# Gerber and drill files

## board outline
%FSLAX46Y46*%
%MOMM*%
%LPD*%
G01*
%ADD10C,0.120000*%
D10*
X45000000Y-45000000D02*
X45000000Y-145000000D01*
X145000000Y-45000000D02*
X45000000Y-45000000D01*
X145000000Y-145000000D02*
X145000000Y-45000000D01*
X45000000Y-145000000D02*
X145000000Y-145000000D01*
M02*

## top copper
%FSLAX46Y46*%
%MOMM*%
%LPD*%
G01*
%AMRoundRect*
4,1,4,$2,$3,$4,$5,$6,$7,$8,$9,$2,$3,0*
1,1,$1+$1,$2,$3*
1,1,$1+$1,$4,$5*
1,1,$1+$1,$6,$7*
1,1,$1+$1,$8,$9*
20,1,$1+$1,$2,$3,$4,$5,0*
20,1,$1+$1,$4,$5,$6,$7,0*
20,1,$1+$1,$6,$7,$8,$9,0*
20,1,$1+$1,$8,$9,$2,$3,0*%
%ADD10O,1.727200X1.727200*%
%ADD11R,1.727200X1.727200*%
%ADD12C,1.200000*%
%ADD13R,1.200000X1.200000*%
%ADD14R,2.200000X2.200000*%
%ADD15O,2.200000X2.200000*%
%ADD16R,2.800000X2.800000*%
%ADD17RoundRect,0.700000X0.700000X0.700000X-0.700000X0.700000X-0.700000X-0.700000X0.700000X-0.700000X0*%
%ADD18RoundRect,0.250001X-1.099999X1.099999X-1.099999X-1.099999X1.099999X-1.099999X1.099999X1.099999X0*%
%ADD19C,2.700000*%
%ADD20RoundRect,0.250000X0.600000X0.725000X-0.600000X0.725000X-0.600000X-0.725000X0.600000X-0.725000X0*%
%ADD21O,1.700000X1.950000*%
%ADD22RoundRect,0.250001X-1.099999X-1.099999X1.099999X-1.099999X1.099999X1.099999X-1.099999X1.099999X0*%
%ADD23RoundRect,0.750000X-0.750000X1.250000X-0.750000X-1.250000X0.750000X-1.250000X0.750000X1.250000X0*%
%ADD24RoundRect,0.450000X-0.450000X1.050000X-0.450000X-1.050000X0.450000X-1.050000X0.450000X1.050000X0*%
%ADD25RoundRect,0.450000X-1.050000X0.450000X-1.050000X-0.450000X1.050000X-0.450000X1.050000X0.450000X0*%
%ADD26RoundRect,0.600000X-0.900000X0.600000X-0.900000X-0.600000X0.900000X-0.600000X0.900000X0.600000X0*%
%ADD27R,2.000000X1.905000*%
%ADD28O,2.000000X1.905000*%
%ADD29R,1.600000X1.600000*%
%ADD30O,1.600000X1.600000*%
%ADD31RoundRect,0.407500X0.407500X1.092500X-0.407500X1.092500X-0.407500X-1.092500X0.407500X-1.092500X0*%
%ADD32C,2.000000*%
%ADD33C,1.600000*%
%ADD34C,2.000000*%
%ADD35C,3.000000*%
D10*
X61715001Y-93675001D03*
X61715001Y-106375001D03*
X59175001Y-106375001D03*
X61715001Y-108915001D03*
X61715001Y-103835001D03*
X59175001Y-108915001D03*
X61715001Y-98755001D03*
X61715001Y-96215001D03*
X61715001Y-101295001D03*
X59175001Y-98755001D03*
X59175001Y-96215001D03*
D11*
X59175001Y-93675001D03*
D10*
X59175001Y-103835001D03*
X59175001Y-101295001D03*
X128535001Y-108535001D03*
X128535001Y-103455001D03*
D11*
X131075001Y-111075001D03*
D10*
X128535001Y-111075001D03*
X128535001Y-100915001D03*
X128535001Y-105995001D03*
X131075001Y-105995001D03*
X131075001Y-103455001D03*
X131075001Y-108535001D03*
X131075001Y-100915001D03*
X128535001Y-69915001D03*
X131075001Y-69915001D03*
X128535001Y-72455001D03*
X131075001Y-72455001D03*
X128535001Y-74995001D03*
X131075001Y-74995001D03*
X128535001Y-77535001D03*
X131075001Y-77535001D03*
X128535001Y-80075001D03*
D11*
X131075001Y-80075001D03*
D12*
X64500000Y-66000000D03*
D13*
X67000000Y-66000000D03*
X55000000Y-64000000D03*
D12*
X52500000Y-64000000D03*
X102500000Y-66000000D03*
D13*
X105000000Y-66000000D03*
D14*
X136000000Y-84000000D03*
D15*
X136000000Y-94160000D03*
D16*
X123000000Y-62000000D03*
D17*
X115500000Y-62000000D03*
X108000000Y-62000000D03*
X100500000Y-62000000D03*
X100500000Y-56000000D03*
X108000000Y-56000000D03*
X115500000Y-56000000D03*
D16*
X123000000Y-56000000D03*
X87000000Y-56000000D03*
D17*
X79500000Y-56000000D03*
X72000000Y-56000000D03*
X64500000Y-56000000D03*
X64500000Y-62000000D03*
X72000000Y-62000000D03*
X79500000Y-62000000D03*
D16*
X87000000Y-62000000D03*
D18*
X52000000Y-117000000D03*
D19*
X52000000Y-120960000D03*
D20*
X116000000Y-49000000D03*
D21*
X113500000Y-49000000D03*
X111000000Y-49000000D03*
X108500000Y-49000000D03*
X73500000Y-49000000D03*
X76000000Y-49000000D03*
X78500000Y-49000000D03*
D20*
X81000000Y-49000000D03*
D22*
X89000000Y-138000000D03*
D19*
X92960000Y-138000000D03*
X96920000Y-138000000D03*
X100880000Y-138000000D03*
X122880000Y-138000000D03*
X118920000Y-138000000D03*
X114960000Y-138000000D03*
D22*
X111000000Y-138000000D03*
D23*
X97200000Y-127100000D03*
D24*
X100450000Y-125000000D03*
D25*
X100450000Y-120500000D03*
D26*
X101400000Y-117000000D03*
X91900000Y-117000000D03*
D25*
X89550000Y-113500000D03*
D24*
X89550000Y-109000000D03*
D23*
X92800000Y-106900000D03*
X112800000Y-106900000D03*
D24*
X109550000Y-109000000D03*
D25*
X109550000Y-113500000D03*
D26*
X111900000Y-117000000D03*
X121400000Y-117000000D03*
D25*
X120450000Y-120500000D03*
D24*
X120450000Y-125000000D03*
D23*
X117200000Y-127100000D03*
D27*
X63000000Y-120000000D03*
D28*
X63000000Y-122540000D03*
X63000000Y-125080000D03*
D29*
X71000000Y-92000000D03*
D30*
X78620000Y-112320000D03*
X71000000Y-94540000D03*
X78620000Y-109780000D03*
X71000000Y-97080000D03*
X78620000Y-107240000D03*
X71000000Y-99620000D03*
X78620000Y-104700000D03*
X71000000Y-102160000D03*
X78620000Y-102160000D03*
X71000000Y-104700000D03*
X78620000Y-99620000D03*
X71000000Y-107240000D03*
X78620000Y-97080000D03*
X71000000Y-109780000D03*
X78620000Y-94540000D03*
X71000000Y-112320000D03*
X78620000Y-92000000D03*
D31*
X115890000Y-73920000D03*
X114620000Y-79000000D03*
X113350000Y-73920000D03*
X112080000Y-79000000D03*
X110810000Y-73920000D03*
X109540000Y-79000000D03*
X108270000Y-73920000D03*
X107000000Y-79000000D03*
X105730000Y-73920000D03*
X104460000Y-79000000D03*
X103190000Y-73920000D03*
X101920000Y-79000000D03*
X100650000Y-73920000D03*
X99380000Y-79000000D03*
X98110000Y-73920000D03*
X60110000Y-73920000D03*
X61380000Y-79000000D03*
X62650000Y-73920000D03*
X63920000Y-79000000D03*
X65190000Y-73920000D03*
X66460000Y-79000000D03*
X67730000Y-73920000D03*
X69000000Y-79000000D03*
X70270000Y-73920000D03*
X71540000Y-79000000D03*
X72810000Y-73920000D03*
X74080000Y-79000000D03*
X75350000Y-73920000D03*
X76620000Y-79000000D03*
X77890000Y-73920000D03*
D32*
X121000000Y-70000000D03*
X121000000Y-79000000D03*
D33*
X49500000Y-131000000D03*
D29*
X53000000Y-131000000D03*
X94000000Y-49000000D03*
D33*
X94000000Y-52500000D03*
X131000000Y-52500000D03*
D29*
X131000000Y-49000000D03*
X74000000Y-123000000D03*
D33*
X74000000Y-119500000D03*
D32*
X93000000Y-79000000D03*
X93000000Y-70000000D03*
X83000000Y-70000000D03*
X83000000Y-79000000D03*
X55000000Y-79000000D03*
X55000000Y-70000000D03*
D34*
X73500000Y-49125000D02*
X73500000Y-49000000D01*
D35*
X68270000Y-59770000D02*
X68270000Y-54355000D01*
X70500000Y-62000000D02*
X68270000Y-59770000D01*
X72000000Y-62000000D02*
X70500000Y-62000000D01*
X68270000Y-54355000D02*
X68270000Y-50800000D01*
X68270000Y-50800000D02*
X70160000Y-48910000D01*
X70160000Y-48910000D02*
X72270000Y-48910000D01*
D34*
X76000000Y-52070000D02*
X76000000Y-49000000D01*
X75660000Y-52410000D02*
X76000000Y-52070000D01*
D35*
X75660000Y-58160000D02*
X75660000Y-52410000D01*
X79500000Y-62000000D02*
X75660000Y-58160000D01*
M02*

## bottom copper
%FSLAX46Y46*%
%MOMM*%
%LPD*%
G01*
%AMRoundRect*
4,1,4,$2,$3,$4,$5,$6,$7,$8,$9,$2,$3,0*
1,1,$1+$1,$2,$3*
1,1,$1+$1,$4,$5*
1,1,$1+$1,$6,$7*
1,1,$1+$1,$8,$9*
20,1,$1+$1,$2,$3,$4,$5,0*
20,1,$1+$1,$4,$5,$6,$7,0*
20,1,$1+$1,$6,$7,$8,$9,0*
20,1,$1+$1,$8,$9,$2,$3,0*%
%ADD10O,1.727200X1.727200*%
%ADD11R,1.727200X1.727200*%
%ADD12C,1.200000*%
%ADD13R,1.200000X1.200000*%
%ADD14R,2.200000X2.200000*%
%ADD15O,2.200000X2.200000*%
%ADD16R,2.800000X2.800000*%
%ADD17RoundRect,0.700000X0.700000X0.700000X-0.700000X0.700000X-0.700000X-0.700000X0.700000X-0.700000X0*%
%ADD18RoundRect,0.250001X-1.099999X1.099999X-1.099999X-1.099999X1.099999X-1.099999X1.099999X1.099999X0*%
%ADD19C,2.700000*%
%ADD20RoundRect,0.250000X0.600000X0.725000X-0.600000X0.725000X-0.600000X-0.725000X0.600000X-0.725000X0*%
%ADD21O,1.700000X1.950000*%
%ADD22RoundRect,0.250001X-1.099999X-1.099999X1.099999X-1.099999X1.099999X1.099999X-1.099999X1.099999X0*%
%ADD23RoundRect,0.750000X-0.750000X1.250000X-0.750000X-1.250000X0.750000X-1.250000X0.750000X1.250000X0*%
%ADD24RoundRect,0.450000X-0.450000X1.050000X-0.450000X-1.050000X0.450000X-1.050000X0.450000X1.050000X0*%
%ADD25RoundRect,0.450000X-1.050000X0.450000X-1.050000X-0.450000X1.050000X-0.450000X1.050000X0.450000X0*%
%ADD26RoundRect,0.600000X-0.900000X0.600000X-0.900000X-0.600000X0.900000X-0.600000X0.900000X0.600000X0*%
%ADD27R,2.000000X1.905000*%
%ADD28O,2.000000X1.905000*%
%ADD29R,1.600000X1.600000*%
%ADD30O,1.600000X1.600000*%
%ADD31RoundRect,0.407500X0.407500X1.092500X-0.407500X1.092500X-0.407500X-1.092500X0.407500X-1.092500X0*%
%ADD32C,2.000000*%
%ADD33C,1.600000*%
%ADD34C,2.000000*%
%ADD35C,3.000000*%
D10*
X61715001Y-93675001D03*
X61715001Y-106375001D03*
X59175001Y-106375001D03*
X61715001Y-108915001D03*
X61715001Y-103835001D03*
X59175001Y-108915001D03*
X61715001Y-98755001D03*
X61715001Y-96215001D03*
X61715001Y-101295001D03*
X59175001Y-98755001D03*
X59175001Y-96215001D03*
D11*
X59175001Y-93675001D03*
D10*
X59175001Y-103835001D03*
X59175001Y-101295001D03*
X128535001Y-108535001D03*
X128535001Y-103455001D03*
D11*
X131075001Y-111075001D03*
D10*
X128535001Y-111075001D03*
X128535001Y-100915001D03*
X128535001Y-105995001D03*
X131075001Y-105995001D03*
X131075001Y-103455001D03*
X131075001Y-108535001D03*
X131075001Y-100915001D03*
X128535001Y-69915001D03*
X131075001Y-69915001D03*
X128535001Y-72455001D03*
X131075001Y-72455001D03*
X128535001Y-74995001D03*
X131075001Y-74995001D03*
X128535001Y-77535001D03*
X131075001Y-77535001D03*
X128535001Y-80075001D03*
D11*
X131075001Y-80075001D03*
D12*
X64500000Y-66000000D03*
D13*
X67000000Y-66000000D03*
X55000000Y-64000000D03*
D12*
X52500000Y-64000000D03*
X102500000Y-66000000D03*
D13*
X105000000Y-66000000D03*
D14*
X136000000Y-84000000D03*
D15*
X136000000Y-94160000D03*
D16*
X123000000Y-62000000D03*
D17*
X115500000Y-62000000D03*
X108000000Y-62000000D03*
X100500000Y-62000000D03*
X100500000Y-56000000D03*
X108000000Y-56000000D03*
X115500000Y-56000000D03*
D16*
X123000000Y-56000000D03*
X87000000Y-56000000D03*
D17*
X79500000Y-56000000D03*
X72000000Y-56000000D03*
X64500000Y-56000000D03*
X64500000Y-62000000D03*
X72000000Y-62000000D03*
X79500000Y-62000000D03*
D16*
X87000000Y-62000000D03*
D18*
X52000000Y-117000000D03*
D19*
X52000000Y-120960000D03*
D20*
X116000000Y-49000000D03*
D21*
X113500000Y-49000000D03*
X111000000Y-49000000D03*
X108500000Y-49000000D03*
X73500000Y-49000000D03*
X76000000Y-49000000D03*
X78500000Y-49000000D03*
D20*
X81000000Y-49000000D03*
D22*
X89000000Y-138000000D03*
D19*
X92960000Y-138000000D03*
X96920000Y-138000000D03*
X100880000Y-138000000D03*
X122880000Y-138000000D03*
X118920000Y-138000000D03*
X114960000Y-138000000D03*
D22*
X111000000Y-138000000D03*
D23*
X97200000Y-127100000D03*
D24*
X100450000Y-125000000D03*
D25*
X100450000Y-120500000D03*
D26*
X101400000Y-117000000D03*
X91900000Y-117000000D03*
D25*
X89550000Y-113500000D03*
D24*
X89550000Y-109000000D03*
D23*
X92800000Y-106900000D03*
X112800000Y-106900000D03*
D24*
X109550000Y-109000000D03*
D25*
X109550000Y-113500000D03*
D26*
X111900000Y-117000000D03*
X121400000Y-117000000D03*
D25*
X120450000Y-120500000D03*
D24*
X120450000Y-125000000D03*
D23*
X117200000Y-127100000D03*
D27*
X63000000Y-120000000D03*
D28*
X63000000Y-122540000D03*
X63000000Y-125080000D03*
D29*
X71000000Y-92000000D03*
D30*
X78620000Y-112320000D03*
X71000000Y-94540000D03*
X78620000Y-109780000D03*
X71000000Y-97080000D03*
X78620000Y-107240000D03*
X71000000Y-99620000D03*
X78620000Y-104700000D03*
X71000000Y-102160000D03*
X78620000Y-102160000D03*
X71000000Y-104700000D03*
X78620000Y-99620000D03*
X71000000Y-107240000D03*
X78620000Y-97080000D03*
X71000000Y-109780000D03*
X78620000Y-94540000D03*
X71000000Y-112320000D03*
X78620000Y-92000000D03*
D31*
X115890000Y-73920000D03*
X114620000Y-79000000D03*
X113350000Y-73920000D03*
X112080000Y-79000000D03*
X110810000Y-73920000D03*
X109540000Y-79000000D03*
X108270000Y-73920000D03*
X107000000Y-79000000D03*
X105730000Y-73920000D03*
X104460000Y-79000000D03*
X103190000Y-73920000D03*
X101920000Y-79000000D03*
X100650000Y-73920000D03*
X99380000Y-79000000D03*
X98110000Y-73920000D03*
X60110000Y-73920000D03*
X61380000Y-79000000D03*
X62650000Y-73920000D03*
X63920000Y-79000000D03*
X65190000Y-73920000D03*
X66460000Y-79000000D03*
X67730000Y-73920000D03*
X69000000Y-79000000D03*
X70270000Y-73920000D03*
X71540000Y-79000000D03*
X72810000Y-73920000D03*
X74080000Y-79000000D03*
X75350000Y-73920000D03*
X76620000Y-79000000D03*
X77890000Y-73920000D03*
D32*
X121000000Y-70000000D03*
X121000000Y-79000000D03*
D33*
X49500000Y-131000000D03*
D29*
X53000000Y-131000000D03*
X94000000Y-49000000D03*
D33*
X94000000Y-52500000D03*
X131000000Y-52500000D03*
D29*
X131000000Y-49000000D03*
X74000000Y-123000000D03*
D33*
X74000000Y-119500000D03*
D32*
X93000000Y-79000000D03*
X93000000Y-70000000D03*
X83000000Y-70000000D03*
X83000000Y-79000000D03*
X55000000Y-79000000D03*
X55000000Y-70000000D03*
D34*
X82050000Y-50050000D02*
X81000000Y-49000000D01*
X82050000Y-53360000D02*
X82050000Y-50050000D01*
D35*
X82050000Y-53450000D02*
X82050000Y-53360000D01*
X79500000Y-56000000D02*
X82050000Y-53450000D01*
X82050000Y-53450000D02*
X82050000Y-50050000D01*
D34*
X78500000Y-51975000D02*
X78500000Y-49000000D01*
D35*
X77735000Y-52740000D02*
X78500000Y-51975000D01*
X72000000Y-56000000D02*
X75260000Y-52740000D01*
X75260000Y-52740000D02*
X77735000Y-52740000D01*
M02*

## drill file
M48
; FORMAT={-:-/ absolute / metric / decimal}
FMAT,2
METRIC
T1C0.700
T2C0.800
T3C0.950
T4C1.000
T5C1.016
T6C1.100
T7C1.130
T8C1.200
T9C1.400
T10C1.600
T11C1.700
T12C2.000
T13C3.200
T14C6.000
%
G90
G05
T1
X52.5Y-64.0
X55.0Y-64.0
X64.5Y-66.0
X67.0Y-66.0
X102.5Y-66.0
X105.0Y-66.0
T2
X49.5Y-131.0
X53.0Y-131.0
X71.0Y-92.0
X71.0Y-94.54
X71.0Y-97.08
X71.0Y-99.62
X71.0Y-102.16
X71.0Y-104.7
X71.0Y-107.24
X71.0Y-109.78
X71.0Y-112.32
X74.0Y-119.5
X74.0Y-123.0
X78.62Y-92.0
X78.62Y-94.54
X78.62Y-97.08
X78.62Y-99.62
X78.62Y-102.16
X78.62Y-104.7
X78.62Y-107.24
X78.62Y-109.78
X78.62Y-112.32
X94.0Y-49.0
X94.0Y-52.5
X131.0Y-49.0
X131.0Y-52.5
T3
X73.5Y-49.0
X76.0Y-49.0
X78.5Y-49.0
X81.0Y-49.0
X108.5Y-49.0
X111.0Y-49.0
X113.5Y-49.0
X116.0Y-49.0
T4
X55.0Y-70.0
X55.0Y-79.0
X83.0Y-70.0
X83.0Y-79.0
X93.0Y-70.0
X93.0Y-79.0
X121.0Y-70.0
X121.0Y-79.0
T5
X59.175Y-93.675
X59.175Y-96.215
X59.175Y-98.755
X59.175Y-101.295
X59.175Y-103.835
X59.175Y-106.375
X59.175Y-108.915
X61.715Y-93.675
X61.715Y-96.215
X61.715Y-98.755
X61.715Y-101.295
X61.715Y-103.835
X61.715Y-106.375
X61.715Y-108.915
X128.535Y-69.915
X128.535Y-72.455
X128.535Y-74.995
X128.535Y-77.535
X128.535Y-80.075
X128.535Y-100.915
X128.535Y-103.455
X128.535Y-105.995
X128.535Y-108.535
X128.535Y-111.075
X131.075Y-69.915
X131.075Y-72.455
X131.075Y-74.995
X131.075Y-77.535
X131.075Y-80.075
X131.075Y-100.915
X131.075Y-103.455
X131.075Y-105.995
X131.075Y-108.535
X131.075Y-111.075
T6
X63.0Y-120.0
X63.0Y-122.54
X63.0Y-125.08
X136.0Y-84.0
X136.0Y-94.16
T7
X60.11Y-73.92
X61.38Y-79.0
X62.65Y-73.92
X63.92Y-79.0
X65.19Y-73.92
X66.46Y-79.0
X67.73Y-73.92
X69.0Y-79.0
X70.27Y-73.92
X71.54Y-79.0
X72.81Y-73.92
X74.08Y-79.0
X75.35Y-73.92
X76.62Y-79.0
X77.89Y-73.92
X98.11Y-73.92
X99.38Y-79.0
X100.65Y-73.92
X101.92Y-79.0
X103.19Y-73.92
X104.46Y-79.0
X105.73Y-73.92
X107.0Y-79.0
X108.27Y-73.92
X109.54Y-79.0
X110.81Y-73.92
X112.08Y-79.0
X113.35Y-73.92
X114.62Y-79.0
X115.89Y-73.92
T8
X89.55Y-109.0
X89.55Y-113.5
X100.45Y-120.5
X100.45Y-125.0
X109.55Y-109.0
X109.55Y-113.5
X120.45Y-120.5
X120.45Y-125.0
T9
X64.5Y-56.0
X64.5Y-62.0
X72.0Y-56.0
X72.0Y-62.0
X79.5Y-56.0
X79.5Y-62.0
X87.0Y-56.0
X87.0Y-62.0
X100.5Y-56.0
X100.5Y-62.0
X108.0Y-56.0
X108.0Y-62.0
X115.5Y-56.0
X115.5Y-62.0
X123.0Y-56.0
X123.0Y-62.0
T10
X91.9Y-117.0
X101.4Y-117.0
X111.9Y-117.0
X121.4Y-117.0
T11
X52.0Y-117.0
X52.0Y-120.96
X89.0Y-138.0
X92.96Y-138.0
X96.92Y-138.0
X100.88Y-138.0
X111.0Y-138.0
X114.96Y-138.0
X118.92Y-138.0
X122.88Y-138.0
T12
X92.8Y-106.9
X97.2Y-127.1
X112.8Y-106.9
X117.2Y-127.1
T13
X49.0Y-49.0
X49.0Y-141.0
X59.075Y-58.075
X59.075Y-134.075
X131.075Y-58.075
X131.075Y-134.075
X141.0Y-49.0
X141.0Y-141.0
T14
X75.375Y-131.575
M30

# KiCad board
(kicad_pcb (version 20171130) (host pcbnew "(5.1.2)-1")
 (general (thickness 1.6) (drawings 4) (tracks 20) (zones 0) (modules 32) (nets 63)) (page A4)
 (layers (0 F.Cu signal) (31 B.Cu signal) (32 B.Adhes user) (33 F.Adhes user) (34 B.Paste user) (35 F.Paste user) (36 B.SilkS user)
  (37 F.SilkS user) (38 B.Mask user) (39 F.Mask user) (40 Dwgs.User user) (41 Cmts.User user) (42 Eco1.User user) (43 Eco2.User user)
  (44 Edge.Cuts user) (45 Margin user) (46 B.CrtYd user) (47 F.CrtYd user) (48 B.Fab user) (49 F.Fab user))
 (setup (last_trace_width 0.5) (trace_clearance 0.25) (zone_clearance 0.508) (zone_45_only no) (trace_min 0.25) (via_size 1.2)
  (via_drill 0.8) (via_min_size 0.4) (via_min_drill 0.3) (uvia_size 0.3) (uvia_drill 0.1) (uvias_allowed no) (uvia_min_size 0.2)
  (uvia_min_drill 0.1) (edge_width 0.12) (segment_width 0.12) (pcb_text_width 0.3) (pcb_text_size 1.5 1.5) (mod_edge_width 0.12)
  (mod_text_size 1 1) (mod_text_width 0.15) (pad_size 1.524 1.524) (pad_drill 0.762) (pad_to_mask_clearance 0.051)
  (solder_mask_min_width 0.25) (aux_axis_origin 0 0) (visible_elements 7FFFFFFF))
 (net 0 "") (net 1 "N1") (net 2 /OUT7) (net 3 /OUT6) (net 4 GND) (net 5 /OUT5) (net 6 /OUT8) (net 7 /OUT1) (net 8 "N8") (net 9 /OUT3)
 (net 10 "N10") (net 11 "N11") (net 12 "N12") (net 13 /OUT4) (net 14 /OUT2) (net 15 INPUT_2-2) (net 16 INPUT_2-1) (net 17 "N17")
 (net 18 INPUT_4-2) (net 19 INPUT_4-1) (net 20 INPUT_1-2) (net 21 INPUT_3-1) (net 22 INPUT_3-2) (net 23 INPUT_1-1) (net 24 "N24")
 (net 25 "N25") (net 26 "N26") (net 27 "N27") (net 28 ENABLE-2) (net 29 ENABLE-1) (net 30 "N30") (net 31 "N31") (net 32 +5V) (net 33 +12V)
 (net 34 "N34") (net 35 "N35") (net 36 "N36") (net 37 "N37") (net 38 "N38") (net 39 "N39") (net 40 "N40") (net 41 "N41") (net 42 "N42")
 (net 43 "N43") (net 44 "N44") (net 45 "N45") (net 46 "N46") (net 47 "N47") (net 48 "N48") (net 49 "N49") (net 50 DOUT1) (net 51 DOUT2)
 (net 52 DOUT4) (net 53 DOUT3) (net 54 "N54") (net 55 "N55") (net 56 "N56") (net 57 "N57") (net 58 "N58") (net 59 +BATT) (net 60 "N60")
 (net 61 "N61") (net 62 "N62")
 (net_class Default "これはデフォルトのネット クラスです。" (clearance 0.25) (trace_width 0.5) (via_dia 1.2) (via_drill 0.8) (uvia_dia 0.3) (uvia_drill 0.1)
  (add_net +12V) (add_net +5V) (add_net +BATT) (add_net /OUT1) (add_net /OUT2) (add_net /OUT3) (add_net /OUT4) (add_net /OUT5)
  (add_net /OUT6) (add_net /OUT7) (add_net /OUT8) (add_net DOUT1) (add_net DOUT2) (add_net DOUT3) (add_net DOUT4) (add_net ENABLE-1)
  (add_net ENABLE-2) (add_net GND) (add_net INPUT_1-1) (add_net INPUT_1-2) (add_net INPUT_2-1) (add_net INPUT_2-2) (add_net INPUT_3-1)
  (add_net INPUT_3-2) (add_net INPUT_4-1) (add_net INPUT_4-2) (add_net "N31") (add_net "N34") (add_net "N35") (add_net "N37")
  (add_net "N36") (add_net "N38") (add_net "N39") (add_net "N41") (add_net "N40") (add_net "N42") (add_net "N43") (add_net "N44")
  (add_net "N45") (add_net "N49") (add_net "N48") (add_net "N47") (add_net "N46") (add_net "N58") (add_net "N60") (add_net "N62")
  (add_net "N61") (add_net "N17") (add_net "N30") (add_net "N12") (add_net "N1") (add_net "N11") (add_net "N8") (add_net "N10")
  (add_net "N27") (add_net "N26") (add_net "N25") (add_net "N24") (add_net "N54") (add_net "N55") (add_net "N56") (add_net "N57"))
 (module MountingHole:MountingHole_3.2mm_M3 (layer F.Cu) (at 141 49)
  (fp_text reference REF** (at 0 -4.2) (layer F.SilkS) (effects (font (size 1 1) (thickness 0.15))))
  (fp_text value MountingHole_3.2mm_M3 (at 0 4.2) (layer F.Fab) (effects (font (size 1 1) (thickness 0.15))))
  (pad 1 np_thru_hole circle (at 0 0) (size 3.2 3.2) (drill 3.2) (layers *.Cu *.Mask)))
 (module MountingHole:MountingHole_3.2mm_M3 (layer F.Cu) (at 141 141)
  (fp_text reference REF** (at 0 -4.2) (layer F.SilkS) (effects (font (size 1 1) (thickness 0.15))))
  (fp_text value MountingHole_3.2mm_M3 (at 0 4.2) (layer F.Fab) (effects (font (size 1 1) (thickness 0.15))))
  (pad 1 np_thru_hole circle (at 0 0) (size 3.2 3.2) (drill 3.2) (layers *.Cu *.Mask)))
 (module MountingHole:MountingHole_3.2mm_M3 (layer F.Cu) (at 49 141)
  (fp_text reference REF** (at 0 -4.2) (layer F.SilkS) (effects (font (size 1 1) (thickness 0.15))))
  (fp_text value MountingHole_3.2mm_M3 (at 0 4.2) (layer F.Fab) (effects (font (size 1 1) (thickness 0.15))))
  (pad 1 np_thru_hole circle (at 0 0) (size 3.2 3.2) (drill 3.2) (layers *.Cu *.Mask)))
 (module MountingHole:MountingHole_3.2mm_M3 (layer F.Cu) (at 49 49)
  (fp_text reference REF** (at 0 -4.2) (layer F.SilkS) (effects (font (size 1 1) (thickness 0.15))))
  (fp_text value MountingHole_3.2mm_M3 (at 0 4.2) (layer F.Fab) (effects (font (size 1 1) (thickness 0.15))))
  (pad 1 np_thru_hole circle (at 0 0) (size 3.2 3.2) (drill 3.2) (layers *.Cu *.Mask)))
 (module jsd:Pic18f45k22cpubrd (layer F.Cu) (at 59.075001 58.075001)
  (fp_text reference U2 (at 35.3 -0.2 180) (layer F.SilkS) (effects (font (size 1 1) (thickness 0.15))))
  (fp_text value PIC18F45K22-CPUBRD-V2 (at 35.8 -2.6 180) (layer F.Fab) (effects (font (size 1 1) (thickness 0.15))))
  (pad "" np_thru_hole circle (at 16.3 73.5) (size 6 6) (drill 6) (layers *.Cu *.Mask))
  (pad "" np_thru_hole circle (at 72 76) (size 3.2 3.2) (drill 3.2) (layers *.Cu *.Mask))
  (pad "" np_thru_hole circle (at 72 0) (size 3.2 3.2) (drill 3.2) (layers *.Cu *.Mask))
  (pad "" np_thru_hole circle (at 0 0) (size 3.2 3.2) (drill 3.2) (layers *.Cu *.Mask))
  (pad "" np_thru_hole circle (at 0 76) (size 3.2 3.2) (drill 3.2) (layers *.Cu *.Mask))
  (pad 22 thru_hole oval (at 2.64 35.6) (size 1.7272 1.7272) (drill 1.016) (layers *.Cu *.Mask) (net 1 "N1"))
  (pad 32 thru_hole oval (at 2.64 48.3) (size 1.7272 1.7272) (drill 1.016) (layers *.Cu *.Mask) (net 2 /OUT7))
  (pad 31 thru_hole oval (at 0.1 48.3) (size 1.7272 1.7272) (drill 1.016) (layers *.Cu *.Mask) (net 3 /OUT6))
  (pad 34 thru_hole oval (at 2.64 50.84) (size 1.7272 1.7272) (drill 1.016) (layers *.Cu *.Mask) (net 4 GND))
  (pad 30 thru_hole oval (at 2.64 45.76) (size 1.7272 1.7272) (drill 1.016) (layers *.Cu *.Mask) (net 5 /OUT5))
  (pad 33 thru_hole oval (at 0.1 50.84) (size 1.7272 1.7272) (drill 1.016) (layers *.Cu *.Mask) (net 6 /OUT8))
  (pad 26 thru_hole oval (at 2.64 40.68) (size 1.7272 1.7272) (drill 1.016) (layers *.Cu *.Mask) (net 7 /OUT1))
  (pad 24 thru_hole oval (at 2.64 38.14) (size 1.7272 1.7272) (drill 1.016) (layers *.Cu *.Mask) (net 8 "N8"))
  (pad 28 thru_hole oval (at 2.64 43.22) (size 1.7272 1.7272) (drill 1.016) (layers *.Cu *.Mask) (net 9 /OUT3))
  (pad 25 thru_hole oval (at 0.1 40.68) (size 1.7272 1.7272) (drill 1.016) (layers *.Cu *.Mask) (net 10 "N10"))
  (pad 23 thru_hole oval (at 0.1 38.14) (size 1.7272 1.7272) (drill 1.016) (layers *.Cu *.Mask) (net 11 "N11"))
  (pad 21 thru_hole rect (at 0.1 35.6) (size 1.7272 1.7272) (drill 1.016) (layers *.Cu *.Mask) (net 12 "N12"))
  (pad 29 thru_hole oval (at 0.1 45.76) (size 1.7272 1.7272) (drill 1.016) (layers *.Cu *.Mask) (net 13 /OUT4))
  (pad 27 thru_hole oval (at 0.1 43.22) (size 1.7272 1.7272) (drill 1.016) (layers *.Cu *.Mask) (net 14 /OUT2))
  (pad 14 thru_hole oval (at 69.46 50.46 180) (size 1.7272 1.7272) (drill 1.016) (layers *.Cu *.Mask) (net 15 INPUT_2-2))
  (pad 18 thru_hole oval (at 69.46 45.38 180) (size 1.7272 1.7272) (drill 1.016) (layers *.Cu *.Mask) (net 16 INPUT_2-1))
  (pad 11 thru_hole rect (at 72 53 180) (size 1.7272 1.7272) (drill 1.016) (layers *.Cu *.Mask) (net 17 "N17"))
  (pad 12 thru_hole oval (at 69.46 53 180) (size 1.7272 1.7272) (drill 1.016) (layers *.Cu *.Mask) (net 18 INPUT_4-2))
  (pad 20 thru_hole oval (at 69.46 42.84 180) (size 1.7272 1.7272) (drill 1.016) (layers *.Cu *.Mask) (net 4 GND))
  (pad 16 thru_hole oval (at 69.46 47.92 180) (size 1.7272 1.7272) (drill 1.016) (layers *.Cu *.Mask) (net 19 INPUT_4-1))
  (pad 15 thru_hole oval (at 72 47.92 180) (size 1.7272 1.7272) (drill 1.016) (layers *.Cu *.Mask) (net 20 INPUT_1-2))
  (pad 17 thru_hole oval (at 72 45.38 180) (size 1.7272 1.7272) (drill 1.016) (layers *.Cu *.Mask) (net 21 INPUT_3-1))
  (pad 13 thru_hole oval (at 72 50.46 180) (size 1.7272 1.7272) (drill 1.016) (layers *.Cu *.Mask) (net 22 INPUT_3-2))
  (pad 19 thru_hole oval (at 72 42.84 180) (size 1.7272 1.7272) (drill 1.016) (layers *.Cu *.Mask) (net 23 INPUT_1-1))
  (pad 10 thru_hole oval (at 69.46 11.84 180) (size 1.7272 1.7272) (drill 1.016) (layers *.Cu *.Mask) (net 4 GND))
  (pad 9 thru_hole oval (at 72 11.84 180) (size 1.7272 1.7272) (drill 1.016) (layers *.Cu *.Mask) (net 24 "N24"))
  (pad 8 thru_hole oval (at 69.46 14.38 180) (size 1.7272 1.7272) (drill 1.016) (layers *.Cu *.Mask) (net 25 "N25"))
  (pad 7 thru_hole oval (at 72 14.38 180) (size 1.7272 1.7272) (drill 1.016) (layers *.Cu *.Mask) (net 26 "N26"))
  (pad 6 thru_hole oval (at 69.46 16.92 180) (size 1.7272 1.7272) (drill 1.016) (layers *.Cu *.Mask))
  (pad 5 thru_hole oval (at 72 16.92 180) (size 1.7272 1.7272) (drill 1.016) (layers *.Cu *.Mask) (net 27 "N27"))
  (pad 4 thru_hole oval (at 69.46 19.46 180) (size 1.7272 1.7272) (drill 1.016) (layers *.Cu *.Mask) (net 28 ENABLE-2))
  (pad 3 thru_hole oval (at 72 19.46 180) (size 1.7272 1.7272) (drill 1.016) (layers *.Cu *.Mask) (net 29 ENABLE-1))
  (pad 2 thru_hole oval (at 69.46 22 180) (size 1.7272 1.7272) (drill 1.016) (layers *.Cu *.Mask) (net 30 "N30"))
  (pad 1 thru_hole rect (at 72 22 180) (size 1.7272 1.7272) (drill 1.016) (layers *.Cu *.Mask) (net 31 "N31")))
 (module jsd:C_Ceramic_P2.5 (layer F.Cu) (at 67 66 180)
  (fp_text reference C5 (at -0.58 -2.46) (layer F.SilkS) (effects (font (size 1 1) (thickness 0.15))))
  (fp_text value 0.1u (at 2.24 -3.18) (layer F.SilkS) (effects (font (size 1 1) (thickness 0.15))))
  (pad 2 thru_hole circle (at 2.5 0 180) (size 1.2 1.2) (drill 0.7) (layers *.Cu *.Mask F.SilkS) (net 4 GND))
  (pad 1 thru_hole rect (at 0 0 180) (size 1.2 1.2) (drill 0.7) (layers *.Cu *.Mask F.SilkS) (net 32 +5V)))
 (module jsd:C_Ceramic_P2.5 (layer F.Cu) (at 55 64 180)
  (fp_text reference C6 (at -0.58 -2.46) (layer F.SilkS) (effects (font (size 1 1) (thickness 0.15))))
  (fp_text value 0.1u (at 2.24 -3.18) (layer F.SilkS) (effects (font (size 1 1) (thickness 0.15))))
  (pad 1 thru_hole rect (at 0 0 180) (size 1.2 1.2) (drill 0.7) (layers *.Cu *.Mask F.SilkS) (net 32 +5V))
  (pad 2 thru_hole circle (at 2.5 0 180) (size 1.2 1.2) (drill 0.7) (layers *.Cu *.Mask F.SilkS) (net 4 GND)))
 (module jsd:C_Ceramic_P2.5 (layer F.Cu) (at 105 66 180)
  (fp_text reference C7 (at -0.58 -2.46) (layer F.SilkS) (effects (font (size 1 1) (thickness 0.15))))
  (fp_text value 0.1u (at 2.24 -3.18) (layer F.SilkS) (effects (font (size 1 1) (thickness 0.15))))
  (pad 2 thru_hole circle (at 2.5 0 180) (size 1.2 1.2) (drill 0.7) (layers *.Cu *.Mask F.SilkS) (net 4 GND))
  (pad 1 thru_hole rect (at 0 0 180) (size 1.2 1.2) (drill 0.7) (layers *.Cu *.Mask F.SilkS) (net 32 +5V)))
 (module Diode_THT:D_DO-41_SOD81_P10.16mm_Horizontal (layer F.Cu) (at 136 84 270)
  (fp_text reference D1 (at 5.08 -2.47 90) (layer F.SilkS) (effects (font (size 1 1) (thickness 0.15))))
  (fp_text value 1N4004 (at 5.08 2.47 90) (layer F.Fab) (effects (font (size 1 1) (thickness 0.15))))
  (pad 1 thru_hole rect (at 0 0 270) (size 2.2 2.2) (drill 1.1) (layers *.Cu *.Mask) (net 31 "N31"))
  (pad 2 thru_hole oval (at 10.16 0 270) (size 2.2 2.2) (drill 1.1) (layers *.Cu *.Mask) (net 32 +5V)))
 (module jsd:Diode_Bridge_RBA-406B (layer F.Cu) (at 123 62 180)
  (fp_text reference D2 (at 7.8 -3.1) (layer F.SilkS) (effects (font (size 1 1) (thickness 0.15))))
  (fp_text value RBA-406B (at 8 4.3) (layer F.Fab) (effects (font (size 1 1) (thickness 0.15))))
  (pad 1 thru_hole rect (at 0 0 180) (size 2.8 2.8) (drill 1.4) (layers *.Cu *.Mask) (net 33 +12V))
  (pad 2 thru_hole roundrect (at 7.5 0 180) (size 2.8 2.8) (drill 1.4) (layers *.Cu *.Mask) (roundrect_rratio 0.25) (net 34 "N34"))
  (pad 3 thru_hole roundrect (at 15 0 180) (size 2.8 2.8) (drill 1.4) (layers *.Cu *.Mask) (roundrect_rratio 0.25) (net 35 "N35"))
  (pad 4 thru_hole roundrect (at 22.5 0 180) (size 2.8 2.8) (drill 1.4) (layers *.Cu *.Mask) (roundrect_rratio 0.25) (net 4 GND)))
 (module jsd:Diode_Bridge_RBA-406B (layer F.Cu) (at 123 56 180)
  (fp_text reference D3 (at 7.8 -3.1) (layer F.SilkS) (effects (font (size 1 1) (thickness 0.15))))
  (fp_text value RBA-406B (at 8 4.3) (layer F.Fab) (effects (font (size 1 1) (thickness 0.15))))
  (pad 4 thru_hole roundrect (at 22.5 0 180) (size 2.8 2.8) (drill 1.4) (layers *.Cu *.Mask) (roundrect_rratio 0.25) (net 4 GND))
  (pad 3 thru_hole roundrect (at 15 0 180) (size 2.8 2.8) (drill 1.4) (layers *.Cu *.Mask) (roundrect_rratio 0.25) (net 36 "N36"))
  (pad 2 thru_hole roundrect (at 7.5 0 180) (size 2.8 2.8) (drill 1.4) (layers *.Cu *.Mask) (roundrect_rratio 0.25) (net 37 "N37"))
  (pad 1 thru_hole rect (at 0 0 180) (size 2.8 2.8) (drill 1.4) (layers *.Cu *.Mask) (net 33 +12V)))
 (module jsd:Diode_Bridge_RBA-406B (layer F.Cu) (at 87 56 180)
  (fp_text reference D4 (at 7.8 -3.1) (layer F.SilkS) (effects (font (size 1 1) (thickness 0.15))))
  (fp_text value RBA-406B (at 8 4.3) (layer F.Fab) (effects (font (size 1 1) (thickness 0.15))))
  (pad 1 thru_hole rect (at 0 0 180) (size 2.8 2.8) (drill 1.4) (layers *.Cu *.Mask) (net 33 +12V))
  (pad 2 thru_hole roundrect (at 7.5 0 180) (size 2.8 2.8) (drill 1.4) (layers *.Cu *.Mask) (roundrect_rratio 0.25) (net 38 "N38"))
  (pad 3 thru_hole roundrect (at 15 0 180) (size 2.8 2.8) (drill 1.4) (layers *.Cu *.Mask) (roundrect_rratio 0.25) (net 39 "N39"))
  (pad 4 thru_hole roundrect (at 22.5 0 180) (size 2.8 2.8) (drill 1.4) (layers *.Cu *.Mask) (roundrect_rratio 0.25) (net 4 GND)))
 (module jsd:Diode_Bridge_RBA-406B (layer F.Cu) (at 87 62 180)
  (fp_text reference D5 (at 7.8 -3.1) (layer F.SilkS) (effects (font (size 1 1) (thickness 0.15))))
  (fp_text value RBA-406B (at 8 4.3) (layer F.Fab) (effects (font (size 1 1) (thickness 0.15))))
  (pad 4 thru_hole roundrect (at 22.5 0 180) (size 2.8 2.8) (drill 1.4) (layers *.Cu *.Mask) (roundrect_rratio 0.25) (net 4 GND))
  (pad 3 thru_hole roundrect (at 15 0 180) (size 2.8 2.8) (drill 1.4) (layers *.Cu *.Mask) (roundrect_rratio 0.25) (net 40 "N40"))
  (pad 2 thru_hole roundrect (at 7.5 0 180) (size 2.8 2.8) (drill 1.4) (layers *.Cu *.Mask) (roundrect_rratio 0.25) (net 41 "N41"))
  (pad 1 thru_hole rect (at 0 0 180) (size 2.8 2.8) (drill 1.4) (layers *.Cu *.Mask) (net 33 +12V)))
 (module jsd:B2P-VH (layer F.Cu) (at 52 117 270)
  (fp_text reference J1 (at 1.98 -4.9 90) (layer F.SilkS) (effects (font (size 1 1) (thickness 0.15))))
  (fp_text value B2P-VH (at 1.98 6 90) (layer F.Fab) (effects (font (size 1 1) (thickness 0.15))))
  (pad 1 thru_hole roundrect (at 0 0 270) (size 2.7 2.7) (drill 1.7) (layers *.Cu *.Mask) (roundrect_rratio 0.09259299999999999)
   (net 33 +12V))
  (pad 2 thru_hole circle (at 3.96 0 270) (size 2.7 2.7) (drill 1.7) (layers *.Cu *.Mask) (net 4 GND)))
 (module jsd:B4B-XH (layer F.Cu) (at 116 49 180)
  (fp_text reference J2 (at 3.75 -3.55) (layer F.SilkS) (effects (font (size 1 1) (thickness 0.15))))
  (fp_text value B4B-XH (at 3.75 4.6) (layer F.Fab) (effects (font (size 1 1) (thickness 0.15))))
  (pad 1 thru_hole roundrect (at 0 0 180) (size 1.7 1.95) (drill 0.95) (layers *.Cu *.Mask) (roundrect_rratio 0.147059) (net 34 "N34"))
  (pad 2 thru_hole oval (at 2.5 0 180) (size 1.7 1.95) (drill 0.95) (layers *.Cu *.Mask) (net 35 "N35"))
  (pad 3 thru_hole oval (at 5 0 180) (size 1.7 1.95) (drill 0.95) (layers *.Cu *.Mask) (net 37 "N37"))
  (pad 4 thru_hole oval (at 7.5 0 180) (size 1.7 1.95) (drill 0.95) (layers *.Cu *.Mask) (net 36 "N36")))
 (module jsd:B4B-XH (layer F.Cu) (at 81 49 180)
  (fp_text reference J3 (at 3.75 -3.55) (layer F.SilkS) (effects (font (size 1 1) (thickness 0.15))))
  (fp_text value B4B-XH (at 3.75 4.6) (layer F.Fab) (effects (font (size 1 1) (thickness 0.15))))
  (pad 4 thru_hole oval (at 7.5 0 180) (size 1.7 1.95) (drill 0.95) (layers *.Cu *.Mask) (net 40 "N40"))
  (pad 3 thru_hole oval (at 5 0 180) (size 1.7 1.95) (drill 0.95) (layers *.Cu *.Mask) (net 41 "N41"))
  (pad 2 thru_hole oval (at 2.5 0 180) (size 1.7 1.95) (drill 0.95) (layers *.Cu *.Mask) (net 39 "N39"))
  (pad 1 thru_hole roundrect (at 0 0 180) (size 1.7 1.95) (drill 0.95) (layers *.Cu *.Mask) (roundrect_rratio 0.147059) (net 38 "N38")))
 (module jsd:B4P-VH (layer F.Cu) (at 89 138)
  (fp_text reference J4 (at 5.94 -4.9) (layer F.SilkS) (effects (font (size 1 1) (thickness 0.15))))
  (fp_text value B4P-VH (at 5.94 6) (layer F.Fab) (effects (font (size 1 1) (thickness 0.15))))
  (pad 1 thru_hole roundrect (at 0 0) (size 2.7 2.7) (drill 1.7) (layers *.Cu *.Mask) (roundrect_rratio 0.09259299999999999) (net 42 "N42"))
  (pad 2 thru_hole circle (at 3.96 0) (size 2.7 2.7) (drill 1.7) (layers *.Cu *.Mask) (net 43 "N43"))
  (pad 3 thru_hole circle (at 7.92 0) (size 2.7 2.7) (drill 1.7) (layers *.Cu *.Mask) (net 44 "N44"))
  (pad 4 thru_hole circle (at 11.88 0) (size 2.7 2.7) (drill 1.7) (layers *.Cu *.Mask) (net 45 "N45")))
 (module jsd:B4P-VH (layer F.Cu) (at 111 138)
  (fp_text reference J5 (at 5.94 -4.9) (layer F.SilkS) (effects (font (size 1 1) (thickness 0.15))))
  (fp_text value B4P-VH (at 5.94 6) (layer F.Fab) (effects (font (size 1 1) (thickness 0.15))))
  (pad 4 thru_hole circle (at 11.88 0) (size 2.7 2.7) (drill 1.7) (layers *.Cu *.Mask) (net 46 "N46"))
  (pad 3 thru_hole circle (at 7.92 0) (size 2.7 2.7) (drill 1.7) (layers *.Cu *.Mask) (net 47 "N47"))
  (pad 2 thru_hole circle (at 3.96 0) (size 2.7 2.7) (drill 1.7) (layers *.Cu *.Mask) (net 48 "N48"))
  (pad 1 thru_hole roundrect (at 0 0) (size 2.7 2.7) (drill 1.7) (layers *.Cu *.Mask) (roundrect_rratio 0.09259299999999999) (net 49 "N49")))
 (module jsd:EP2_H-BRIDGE (layer F.Cu) (at 95 117 270)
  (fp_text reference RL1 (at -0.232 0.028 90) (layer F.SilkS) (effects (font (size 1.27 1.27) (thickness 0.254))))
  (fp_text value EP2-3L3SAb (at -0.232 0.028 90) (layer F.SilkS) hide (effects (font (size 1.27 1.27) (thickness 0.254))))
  (pad 8 thru_hole roundrect (at 10.1 -2.2 270) (size 4 3) (drill 2) (layers *.Cu *.Mask) (roundrect_rratio 0.25) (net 43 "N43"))
  (pad 7 thru_hole roundrect (at 8 -5.45 270) (size 3 1.8) (drill 1.2) (layers *.Cu *.Mask) (roundrect_rratio 0.25) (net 33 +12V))
  (pad 6 thru_hole roundrect (at 3.5 -5.45 270) (size 1.8 3) (drill 1.2) (layers *.Cu *.Mask) (roundrect_rratio 0.25) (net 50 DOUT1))
  (pad 5 thru_hole roundrect (at 0 -6.4 270) (size 2.4 3) (drill 1.6) (layers *.Cu *.Mask) (roundrect_rratio 0.25) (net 45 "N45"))
  (pad 4 thru_hole roundrect (at 0 3.1 270) (size 2.4 3) (drill 1.6) (layers *.Cu *.Mask) (roundrect_rratio 0.25) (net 42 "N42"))
  (pad 3 thru_hole roundrect (at -3.5 5.45 270) (size 1.8 3) (drill 1.2) (layers *.Cu *.Mask) (roundrect_rratio 0.25) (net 33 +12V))
  (pad 2 thru_hole roundrect (at -8 5.45 270) (size 3 1.8) (drill 1.2) (layers *.Cu *.Mask) (roundrect_rratio 0.25) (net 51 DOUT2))
  (pad 1 thru_hole roundrect (at -10.1 2.2 270) (size 4 3) (drill 2) (layers *.Cu *.Mask) (roundrect_rratio 0.25) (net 44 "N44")))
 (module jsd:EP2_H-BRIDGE (layer F.Cu) (at 115 117 270)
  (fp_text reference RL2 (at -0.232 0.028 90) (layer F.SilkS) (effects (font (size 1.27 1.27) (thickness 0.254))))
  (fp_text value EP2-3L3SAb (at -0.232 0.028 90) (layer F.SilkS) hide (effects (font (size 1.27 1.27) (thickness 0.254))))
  (pad 1 thru_hole roundrect (at -10.1 2.2 270) (size 4 3) (drill 2) (layers *.Cu *.Mask) (roundrect_rratio 0.25) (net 47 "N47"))
  (pad 2 thru_hole roundrect (at -8 5.45 270) (size 3 1.8) (drill 1.2) (layers *.Cu *.Mask) (roundrect_rratio 0.25) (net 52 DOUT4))
  (pad 3 thru_hole roundrect (at -3.5 5.45 270) (size 1.8 3) (drill 1.2) (layers *.Cu *.Mask) (roundrect_rratio 0.25) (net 33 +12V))
  (pad 4 thru_hole roundrect (at 0 3.1 270) (size 2.4 3) (drill 1.6) (layers *.Cu *.Mask) (roundrect_rratio 0.25) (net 49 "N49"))
  (pad 5 thru_hole roundrect (at 0 -6.4 270) (size 2.4 3) (drill 1.6) (layers *.Cu *.Mask) (roundrect_rratio 0.25) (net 46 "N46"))
  (pad 6 thru_hole roundrect (at 3.5 -5.45 270) (size 1.8 3) (drill 1.2) (layers *.Cu *.Mask) (roundrect_rratio 0.25) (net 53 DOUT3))
  (pad 7 thru_hole roundrect (at 8 -5.45 270) (size 3 1.8) (drill 1.2) (layers *.Cu *.Mask) (roundrect_rratio 0.25) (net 33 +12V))
  (pad 8 thru_hole roundrect (at 10.1 -2.2 270) (size 4 3) (drill 2) (layers *.Cu *.Mask) (roundrect_rratio 0.25) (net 48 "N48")))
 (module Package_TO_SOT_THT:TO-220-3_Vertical (layer F.Cu) (at 63 120 270)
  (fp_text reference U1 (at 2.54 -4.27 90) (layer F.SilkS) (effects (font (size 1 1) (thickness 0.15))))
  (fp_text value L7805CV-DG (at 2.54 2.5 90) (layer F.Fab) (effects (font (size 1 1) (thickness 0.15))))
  (pad 1 thru_hole rect (at 0 0 270) (size 1.905 2) (drill 1.1) (layers *.Cu *.Mask) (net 33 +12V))
  (pad 2 thru_hole oval (at 2.54 0 270) (size 1.905 2) (drill 1.1) (layers *.Cu *.Mask) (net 4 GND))
  (pad 3 thru_hole oval (at 5.08 0 270) (size 1.905 2) (drill 1.1) (layers *.Cu *.Mask) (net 32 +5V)))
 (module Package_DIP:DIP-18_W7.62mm (layer F.Cu) (at 71 92)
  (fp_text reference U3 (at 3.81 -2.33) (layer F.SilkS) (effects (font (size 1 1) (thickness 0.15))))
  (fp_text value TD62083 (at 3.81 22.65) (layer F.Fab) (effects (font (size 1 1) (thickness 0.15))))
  (pad 1 thru_hole rect (at 0 0) (size 1.6 1.6) (drill 0.8) (layers *.Cu *.Mask) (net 7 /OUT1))
  (pad 10 thru_hole oval (at 7.62 20.32) (size 1.6 1.6) (drill 0.8) (layers *.Cu *.Mask) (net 33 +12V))
  (pad 2 thru_hole oval (at 0 2.54) (size 1.6 1.6) (drill 0.8) (layers *.Cu *.Mask) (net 14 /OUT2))
  (pad 11 thru_hole oval (at 7.62 17.78) (size 1.6 1.6) (drill 0.8) (layers *.Cu *.Mask) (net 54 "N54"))
  (pad 3 thru_hole oval (at 0 5.08) (size 1.6 1.6) (drill 0.8) (layers *.Cu *.Mask) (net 9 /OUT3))
  (pad 12 thru_hole oval (at 7.62 15.24) (size 1.6 1.6) (drill 0.8) (layers *.Cu *.Mask) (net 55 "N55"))
  (pad 4 thru_hole oval (at 0 7.62) (size 1.6 1.6) (drill 0.8) (layers *.Cu *.Mask) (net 13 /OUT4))
  (pad 13 thru_hole oval (at 7.62 12.7) (size 1.6 1.6) (drill 0.8) (layers *.Cu *.Mask) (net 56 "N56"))
  (pad 5 thru_hole oval (at 0 10.16) (size 1.6 1.6) (drill 0.8) (layers *.Cu *.Mask) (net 5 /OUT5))
  (pad 14 thru_hole oval (at 7.62 10.16) (size 1.6 1.6) (drill 0.8) (layers *.Cu *.Mask) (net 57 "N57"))
  (pad 6 thru_hole oval (at 0 12.7) (size 1.6 1.6) (drill 0.8) (layers *.Cu *.Mask) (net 3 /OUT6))
  (pad 15 thru_hole oval (at 7.62 7.62) (size 1.6 1.6) (drill 0.8) (layers *.Cu *.Mask) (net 52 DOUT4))
  (pad 7 thru_hole oval (at 0 15.24) (size 1.6 1.6) (drill 0.8) (layers *.Cu *.Mask) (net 2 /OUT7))
  (pad 16 thru_hole oval (at 7.62 5.08) (size 1.6 1.6) (drill 0.8) (layers *.Cu *.Mask) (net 53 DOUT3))
  (pad 8 thru_hole oval (at 0 17.78) (size 1.6 1.6) (drill 0.8) (layers *.Cu *.Mask) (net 6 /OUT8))
  (pad 17 thru_hole oval (at 7.62 2.54) (size 1.6 1.6) (drill 0.8) (layers *.Cu *.Mask) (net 51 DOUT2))
  (pad 9 thru_hole oval (at 0 20.32) (size 1.6 1.6) (drill 0.8) (layers *.Cu *.Mask) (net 4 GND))
  (pad 18 thru_hole oval (at 7.62 0) (size 1.6 1.6) (drill 0.8) (layers *.Cu *.Mask) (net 50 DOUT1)))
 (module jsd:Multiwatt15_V (layer F.Cu) (at 107 79 180)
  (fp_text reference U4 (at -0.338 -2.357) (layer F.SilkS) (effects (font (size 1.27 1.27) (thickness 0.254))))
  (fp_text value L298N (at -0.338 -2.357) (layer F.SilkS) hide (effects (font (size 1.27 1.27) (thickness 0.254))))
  (pad 1 thru_hole roundrect (at -8.89 5.08 180) (size 1.63 3) (drill 1.13) (layers *.Cu *.Mask) (roundrect_rratio 0.25) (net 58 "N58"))
  (pad 2 thru_hole roundrect (at -7.62 0 180) (size 1.63 3) (drill 1.13) (layers *.Cu *.Mask) (roundrect_rratio 0.25) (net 34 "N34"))
  (pad 3 thru_hole roundrect (at -6.35 5.08 180) (size 1.63 3) (drill 1.13) (layers *.Cu *.Mask) (roundrect_rratio 0.25) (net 35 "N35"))
  (pad 4 thru_hole roundrect (at -5.08 0 180) (size 1.63 3) (drill 1.13) (layers *.Cu *.Mask) (roundrect_rratio 0.25) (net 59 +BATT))
  (pad 5 thru_hole roundrect (at -3.81 5.08 180) (size 1.63 3) (drill 1.13) (layers *.Cu *.Mask) (roundrect_rratio 0.25) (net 23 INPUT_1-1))
  (pad 6 thru_hole roundrect (at -2.54 0 180) (size 1.63 3) (drill 1.13) (layers *.Cu *.Mask) (roundrect_rratio 0.25) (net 29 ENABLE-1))
  (pad 7 thru_hole roundrect (at -1.27 5.08 180) (size 1.63 3) (drill 1.13) (layers *.Cu *.Mask) (roundrect_rratio 0.25) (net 16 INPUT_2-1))
  (pad 8 thru_hole roundrect (at 0 0 180) (size 1.63 3) (drill 1.13) (layers *.Cu *.Mask) (roundrect_rratio 0.25) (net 4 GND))
  (pad 9 thru_hole roundrect (at 1.27 5.08 180) (size 1.63 3) (drill 1.13) (layers *.Cu *.Mask) (roundrect_rratio 0.25) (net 32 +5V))
  (pad 10 thru_hole roundrect (at 2.54 0 180) (size 1.63 3) (drill 1.13) (layers *.Cu *.Mask) (roundrect_rratio 0.25) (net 21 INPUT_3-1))
  (pad 11 thru_hole roundrect (at 3.81 5.08 180) (size 1.63 3) (drill 1.13) (layers *.Cu *.Mask) (roundrect_rratio 0.25) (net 29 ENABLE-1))
  (pad 12 thru_hole roundrect (at 5.08 0 180) (size 1.63 3) (drill 1.13) (layers *.Cu *.Mask) (roundrect_rratio 0.25) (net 19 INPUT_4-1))
  (pad 13 thru_hole roundrect (at 6.35 5.08 180) (size 1.63 3) (drill 1.13) (layers *.Cu *.Mask) (roundrect_rratio 0.25) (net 37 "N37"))
  (pad 14 thru_hole roundrect (at 7.62 0 180) (size 1.63 3) (drill 1.13) (layers *.Cu *.Mask) (roundrect_rratio 0.25) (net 36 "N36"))
  (pad 15 thru_hole roundrect (at 8.89 5.08 180) (size 1.63 3) (drill 1.13) (layers *.Cu *.Mask) (roundrect_rratio 0.25) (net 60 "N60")))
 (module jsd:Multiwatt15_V (layer F.Cu) (at 69 79 180)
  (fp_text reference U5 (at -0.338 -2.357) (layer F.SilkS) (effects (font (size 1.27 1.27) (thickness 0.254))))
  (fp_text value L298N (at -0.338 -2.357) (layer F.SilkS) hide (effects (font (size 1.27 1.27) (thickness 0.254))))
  (pad 15 thru_hole roundrect (at 8.89 5.08 180) (size 1.63 3) (drill 1.13) (layers *.Cu *.Mask) (roundrect_rratio 0.25) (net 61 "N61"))
  (pad 14 thru_hole roundrect (at 7.62 0 180) (size 1.63 3) (drill 1.13) (layers *.Cu *.Mask) (roundrect_rratio 0.25) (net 40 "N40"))
  (pad 13 thru_hole roundrect (at 6.35 5.08 180) (size 1.63 3) (drill 1.13) (layers *.Cu *.Mask) (roundrect_rratio 0.25) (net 41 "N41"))
  (pad 12 thru_hole roundrect (at 5.08 0 180) (size 1.63 3) (drill 1.13) (layers *.Cu *.Mask) (roundrect_rratio 0.25) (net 18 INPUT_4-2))
  (pad 11 thru_hole roundrect (at 3.81 5.08 180) (size 1.63 3) (drill 1.13) (layers *.Cu *.Mask) (roundrect_rratio 0.25) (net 28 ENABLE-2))
  (pad 10 thru_hole roundrect (at 2.54 0 180) (size 1.63 3) (drill 1.13) (layers *.Cu *.Mask) (roundrect_rratio 0.25) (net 22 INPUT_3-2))
  (pad 9 thru_hole roundrect (at 1.27 5.08 180) (size 1.63 3) (drill 1.13) (layers *.Cu *.Mask) (roundrect_rratio 0.25) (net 32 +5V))
  (pad 8 thru_hole roundrect (at 0 0 180) (size 1.63 3) (drill 1.13) (layers *.Cu *.Mask) (roundrect_rratio 0.25) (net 4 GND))
  (pad 7 thru_hole roundrect (at -1.27 5.08 180) (size 1.63 3) (drill 1.13) (layers *.Cu *.Mask) (roundrect_rratio 0.25) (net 15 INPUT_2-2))
  (pad 6 thru_hole roundrect (at -2.54 0 180) (size 1.63 3) (drill 1.13) (layers *.Cu *.Mask) (roundrect_rratio 0.25) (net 28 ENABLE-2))
  (pad 5 thru_hole roundrect (at -3.81 5.08 180) (size 1.63 3) (drill 1.13) (layers *.Cu *.Mask) (roundrect_rratio 0.25) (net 20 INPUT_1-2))
  (pad 4 thru_hole roundrect (at -5.08 0 180) (size 1.63 3) (drill 1.13) (layers *.Cu *.Mask) (roundrect_rratio 0.25) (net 59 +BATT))
  (pad 3 thru_hole roundrect (at -6.35 5.08 180) (size 1.63 3) (drill 1.13) (layers *.Cu *.Mask) (roundrect_rratio 0.25) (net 39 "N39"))
  (pad 2 thru_hole roundrect (at -7.62 0 180) (size 1.63 3) (drill 1.13) (layers *.Cu *.Mask) (roundrect_rratio 0.25) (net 38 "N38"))
  (pad 1 thru_hole roundrect (at -8.89 5.08 180) (size 1.63 3) (drill 1.13) (layers *.Cu *.Mask) (roundrect_rratio 0.25) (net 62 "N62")))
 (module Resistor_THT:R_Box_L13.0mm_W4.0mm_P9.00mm (layer F.Cu) (at 121 79 90)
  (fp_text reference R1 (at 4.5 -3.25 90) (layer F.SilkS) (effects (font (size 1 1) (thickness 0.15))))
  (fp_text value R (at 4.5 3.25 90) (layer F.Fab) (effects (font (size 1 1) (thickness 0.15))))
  (pad 2 thru_hole circle (at 9 0 90) (size 2 2) (drill 1) (layers *.Cu *.Mask) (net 58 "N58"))
  (pad 1 thru_hole circle (at 0 0 90) (size 2 2) (drill 1) (layers *.Cu *.Mask) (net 4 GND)))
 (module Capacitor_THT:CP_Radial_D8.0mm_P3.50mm (layer F.Cu) (at 53 131 180)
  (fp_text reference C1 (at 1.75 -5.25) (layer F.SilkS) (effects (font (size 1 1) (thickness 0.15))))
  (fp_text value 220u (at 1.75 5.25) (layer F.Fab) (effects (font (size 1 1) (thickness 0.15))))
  (pad 2 thru_hole circle (at 3.5 0 180) (size 1.6 1.6) (drill 0.8) (layers *.Cu *.Mask) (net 4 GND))
  (pad 1 thru_hole rect (at 0 0 180) (size 1.6 1.6) (drill 0.8) (layers *.Cu *.Mask) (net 33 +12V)))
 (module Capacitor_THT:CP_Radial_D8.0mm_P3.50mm (layer F.Cu) (at 94 49 270)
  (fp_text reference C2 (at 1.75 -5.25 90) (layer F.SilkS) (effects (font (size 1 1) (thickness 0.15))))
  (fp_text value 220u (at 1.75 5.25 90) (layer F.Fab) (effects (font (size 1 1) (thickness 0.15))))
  (pad 1 thru_hole rect (at 0 0 270) (size 1.6 1.6) (drill 0.8) (layers *.Cu *.Mask) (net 33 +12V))
  (pad 2 thru_hole circle (at 3.5 0 270) (size 1.6 1.6) (drill 0.8) (layers *.Cu *.Mask) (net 4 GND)))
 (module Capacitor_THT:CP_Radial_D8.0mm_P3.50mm (layer F.Cu) (at 131 49 270)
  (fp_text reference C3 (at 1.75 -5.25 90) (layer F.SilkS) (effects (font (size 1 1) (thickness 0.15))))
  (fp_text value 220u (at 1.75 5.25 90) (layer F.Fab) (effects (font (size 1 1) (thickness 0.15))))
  (pad 2 thru_hole circle (at 3.5 0 270) (size 1.6 1.6) (drill 0.8) (layers *.Cu *.Mask) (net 4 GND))
  (pad 1 thru_hole rect (at 0 0 270) (size 1.6 1.6) (drill 0.8) (layers *.Cu *.Mask) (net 33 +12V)))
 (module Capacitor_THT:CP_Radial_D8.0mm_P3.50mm (layer F.Cu) (at 74 123 90)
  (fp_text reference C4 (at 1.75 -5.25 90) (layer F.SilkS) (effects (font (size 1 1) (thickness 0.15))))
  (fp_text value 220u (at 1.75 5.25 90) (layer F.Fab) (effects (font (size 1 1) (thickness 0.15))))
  (pad 1 thru_hole rect (at 0 0 90) (size 1.6 1.6) (drill 0.8) (layers *.Cu *.Mask) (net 32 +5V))
  (pad 2 thru_hole circle (at 3.5 0 90) (size 1.6 1.6) (drill 0.8) (layers *.Cu *.Mask) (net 4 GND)))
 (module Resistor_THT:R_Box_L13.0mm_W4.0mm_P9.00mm (layer F.Cu) (at 93 79 90)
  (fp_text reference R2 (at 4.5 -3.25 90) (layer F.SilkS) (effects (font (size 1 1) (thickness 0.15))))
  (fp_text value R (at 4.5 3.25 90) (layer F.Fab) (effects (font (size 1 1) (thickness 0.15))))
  (pad 1 thru_hole circle (at 0 0 90) (size 2 2) (drill 1) (layers *.Cu *.Mask) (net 4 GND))
  (pad 2 thru_hole circle (at 9 0 90) (size 2 2) (drill 1) (layers *.Cu *.Mask) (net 60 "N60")))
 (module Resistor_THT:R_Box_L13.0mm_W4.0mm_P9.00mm (layer F.Cu) (at 83 79 90)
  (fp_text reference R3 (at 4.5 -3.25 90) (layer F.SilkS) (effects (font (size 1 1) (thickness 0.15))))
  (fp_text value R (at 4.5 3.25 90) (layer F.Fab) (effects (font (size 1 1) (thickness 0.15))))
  (pad 2 thru_hole circle (at 9 0 90) (size 2 2) (drill 1) (layers *.Cu *.Mask) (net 62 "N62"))
  (pad 1 thru_hole circle (at 0 0 90) (size 2 2) (drill 1) (layers *.Cu *.Mask) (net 4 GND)))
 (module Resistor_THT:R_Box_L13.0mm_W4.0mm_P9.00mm (layer F.Cu) (at 55 79 90)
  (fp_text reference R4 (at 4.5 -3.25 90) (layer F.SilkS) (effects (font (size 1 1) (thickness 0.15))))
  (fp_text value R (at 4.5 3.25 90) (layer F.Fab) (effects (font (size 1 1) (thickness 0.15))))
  (pad 1 thru_hole circle (at 0 0 90) (size 2 2) (drill 1) (layers *.Cu *.Mask) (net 4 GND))
  (pad 2 thru_hole circle (at 9 0 90) (size 2 2) (drill 1) (layers *.Cu *.Mask) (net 61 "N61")))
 (gr_line (start 45 45) (end 45 145) (layer Edge.Cuts) (width 0.12))
 (gr_line (start 145 45) (end 45 45) (layer Edge.Cuts) (width 0.12))
 (gr_line (start 145 145) (end 145 45) (layer Edge.Cuts) (width 0.12))
 (gr_line (start 45 145) (end 145 145) (layer Edge.Cuts) (width 0.12))
 (segment (start 82.05 50.05) (end 81 49) (width 2) (layer B.Cu) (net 38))
 (segment (start 82.05 53.36) (end 82.05 50.05) (width 2) (layer B.Cu) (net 38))
 (segment (start 82.05 53.45) (end 82.05 53.36) (width 3) (layer B.Cu) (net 38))
 (segment (start 79.5 56) (end 82.05 53.45) (width 3) (layer B.Cu) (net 38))
 (segment (start 82.05 53.45) (end 82.05 50.05) (width 3) (layer B.Cu) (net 38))
 (segment (start 78.5 51.975) (end 78.5 49) (width 2) (layer B.Cu) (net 39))
 (segment (start 77.735 52.74) (end 78.5 51.975) (width 3) (layer B.Cu) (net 39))
 (segment (start 72 56) (end 75.26 52.74) (width 3) (layer B.Cu) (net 39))
 (segment (start 75.26 52.74) (end 77.735 52.74) (width 3) (layer B.Cu) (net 39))
 (segment (start 73.5 49.125) (end 73.5 49) (width 2) (layer F.Cu) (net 40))
 (segment (start 68.27 59.77) (end 68.27 54.355) (width 3) (layer F.Cu) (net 40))
 (segment (start 70.5 62) (end 68.27 59.77) (width 3) (layer F.Cu) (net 40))
 (segment (start 72 62) (end 70.5 62) (width 3) (layer F.Cu) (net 40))
 (segment (start 68.27 54.355) (end 68.27 50.8) (width 3) (layer F.Cu) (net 40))
 (segment (start 68.27 50.8) (end 70.16 48.91) (width 3) (layer F.Cu) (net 40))
 (segment (start 70.16 48.91) (end 72.27 48.91) (width 3) (layer F.Cu) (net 40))
 (segment (start 76 52.07) (end 76 49) (width 2) (layer F.Cu) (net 41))
 (segment (start 75.66 52.41) (end 76 52.07) (width 2) (layer F.Cu) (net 41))
 (segment (start 75.66 58.16) (end 75.66 52.41) (width 3) (layer F.Cu) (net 41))
 (segment (start 79.5 62) (end 75.66 58.16) (width 3) (layer F.Cu) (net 41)))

